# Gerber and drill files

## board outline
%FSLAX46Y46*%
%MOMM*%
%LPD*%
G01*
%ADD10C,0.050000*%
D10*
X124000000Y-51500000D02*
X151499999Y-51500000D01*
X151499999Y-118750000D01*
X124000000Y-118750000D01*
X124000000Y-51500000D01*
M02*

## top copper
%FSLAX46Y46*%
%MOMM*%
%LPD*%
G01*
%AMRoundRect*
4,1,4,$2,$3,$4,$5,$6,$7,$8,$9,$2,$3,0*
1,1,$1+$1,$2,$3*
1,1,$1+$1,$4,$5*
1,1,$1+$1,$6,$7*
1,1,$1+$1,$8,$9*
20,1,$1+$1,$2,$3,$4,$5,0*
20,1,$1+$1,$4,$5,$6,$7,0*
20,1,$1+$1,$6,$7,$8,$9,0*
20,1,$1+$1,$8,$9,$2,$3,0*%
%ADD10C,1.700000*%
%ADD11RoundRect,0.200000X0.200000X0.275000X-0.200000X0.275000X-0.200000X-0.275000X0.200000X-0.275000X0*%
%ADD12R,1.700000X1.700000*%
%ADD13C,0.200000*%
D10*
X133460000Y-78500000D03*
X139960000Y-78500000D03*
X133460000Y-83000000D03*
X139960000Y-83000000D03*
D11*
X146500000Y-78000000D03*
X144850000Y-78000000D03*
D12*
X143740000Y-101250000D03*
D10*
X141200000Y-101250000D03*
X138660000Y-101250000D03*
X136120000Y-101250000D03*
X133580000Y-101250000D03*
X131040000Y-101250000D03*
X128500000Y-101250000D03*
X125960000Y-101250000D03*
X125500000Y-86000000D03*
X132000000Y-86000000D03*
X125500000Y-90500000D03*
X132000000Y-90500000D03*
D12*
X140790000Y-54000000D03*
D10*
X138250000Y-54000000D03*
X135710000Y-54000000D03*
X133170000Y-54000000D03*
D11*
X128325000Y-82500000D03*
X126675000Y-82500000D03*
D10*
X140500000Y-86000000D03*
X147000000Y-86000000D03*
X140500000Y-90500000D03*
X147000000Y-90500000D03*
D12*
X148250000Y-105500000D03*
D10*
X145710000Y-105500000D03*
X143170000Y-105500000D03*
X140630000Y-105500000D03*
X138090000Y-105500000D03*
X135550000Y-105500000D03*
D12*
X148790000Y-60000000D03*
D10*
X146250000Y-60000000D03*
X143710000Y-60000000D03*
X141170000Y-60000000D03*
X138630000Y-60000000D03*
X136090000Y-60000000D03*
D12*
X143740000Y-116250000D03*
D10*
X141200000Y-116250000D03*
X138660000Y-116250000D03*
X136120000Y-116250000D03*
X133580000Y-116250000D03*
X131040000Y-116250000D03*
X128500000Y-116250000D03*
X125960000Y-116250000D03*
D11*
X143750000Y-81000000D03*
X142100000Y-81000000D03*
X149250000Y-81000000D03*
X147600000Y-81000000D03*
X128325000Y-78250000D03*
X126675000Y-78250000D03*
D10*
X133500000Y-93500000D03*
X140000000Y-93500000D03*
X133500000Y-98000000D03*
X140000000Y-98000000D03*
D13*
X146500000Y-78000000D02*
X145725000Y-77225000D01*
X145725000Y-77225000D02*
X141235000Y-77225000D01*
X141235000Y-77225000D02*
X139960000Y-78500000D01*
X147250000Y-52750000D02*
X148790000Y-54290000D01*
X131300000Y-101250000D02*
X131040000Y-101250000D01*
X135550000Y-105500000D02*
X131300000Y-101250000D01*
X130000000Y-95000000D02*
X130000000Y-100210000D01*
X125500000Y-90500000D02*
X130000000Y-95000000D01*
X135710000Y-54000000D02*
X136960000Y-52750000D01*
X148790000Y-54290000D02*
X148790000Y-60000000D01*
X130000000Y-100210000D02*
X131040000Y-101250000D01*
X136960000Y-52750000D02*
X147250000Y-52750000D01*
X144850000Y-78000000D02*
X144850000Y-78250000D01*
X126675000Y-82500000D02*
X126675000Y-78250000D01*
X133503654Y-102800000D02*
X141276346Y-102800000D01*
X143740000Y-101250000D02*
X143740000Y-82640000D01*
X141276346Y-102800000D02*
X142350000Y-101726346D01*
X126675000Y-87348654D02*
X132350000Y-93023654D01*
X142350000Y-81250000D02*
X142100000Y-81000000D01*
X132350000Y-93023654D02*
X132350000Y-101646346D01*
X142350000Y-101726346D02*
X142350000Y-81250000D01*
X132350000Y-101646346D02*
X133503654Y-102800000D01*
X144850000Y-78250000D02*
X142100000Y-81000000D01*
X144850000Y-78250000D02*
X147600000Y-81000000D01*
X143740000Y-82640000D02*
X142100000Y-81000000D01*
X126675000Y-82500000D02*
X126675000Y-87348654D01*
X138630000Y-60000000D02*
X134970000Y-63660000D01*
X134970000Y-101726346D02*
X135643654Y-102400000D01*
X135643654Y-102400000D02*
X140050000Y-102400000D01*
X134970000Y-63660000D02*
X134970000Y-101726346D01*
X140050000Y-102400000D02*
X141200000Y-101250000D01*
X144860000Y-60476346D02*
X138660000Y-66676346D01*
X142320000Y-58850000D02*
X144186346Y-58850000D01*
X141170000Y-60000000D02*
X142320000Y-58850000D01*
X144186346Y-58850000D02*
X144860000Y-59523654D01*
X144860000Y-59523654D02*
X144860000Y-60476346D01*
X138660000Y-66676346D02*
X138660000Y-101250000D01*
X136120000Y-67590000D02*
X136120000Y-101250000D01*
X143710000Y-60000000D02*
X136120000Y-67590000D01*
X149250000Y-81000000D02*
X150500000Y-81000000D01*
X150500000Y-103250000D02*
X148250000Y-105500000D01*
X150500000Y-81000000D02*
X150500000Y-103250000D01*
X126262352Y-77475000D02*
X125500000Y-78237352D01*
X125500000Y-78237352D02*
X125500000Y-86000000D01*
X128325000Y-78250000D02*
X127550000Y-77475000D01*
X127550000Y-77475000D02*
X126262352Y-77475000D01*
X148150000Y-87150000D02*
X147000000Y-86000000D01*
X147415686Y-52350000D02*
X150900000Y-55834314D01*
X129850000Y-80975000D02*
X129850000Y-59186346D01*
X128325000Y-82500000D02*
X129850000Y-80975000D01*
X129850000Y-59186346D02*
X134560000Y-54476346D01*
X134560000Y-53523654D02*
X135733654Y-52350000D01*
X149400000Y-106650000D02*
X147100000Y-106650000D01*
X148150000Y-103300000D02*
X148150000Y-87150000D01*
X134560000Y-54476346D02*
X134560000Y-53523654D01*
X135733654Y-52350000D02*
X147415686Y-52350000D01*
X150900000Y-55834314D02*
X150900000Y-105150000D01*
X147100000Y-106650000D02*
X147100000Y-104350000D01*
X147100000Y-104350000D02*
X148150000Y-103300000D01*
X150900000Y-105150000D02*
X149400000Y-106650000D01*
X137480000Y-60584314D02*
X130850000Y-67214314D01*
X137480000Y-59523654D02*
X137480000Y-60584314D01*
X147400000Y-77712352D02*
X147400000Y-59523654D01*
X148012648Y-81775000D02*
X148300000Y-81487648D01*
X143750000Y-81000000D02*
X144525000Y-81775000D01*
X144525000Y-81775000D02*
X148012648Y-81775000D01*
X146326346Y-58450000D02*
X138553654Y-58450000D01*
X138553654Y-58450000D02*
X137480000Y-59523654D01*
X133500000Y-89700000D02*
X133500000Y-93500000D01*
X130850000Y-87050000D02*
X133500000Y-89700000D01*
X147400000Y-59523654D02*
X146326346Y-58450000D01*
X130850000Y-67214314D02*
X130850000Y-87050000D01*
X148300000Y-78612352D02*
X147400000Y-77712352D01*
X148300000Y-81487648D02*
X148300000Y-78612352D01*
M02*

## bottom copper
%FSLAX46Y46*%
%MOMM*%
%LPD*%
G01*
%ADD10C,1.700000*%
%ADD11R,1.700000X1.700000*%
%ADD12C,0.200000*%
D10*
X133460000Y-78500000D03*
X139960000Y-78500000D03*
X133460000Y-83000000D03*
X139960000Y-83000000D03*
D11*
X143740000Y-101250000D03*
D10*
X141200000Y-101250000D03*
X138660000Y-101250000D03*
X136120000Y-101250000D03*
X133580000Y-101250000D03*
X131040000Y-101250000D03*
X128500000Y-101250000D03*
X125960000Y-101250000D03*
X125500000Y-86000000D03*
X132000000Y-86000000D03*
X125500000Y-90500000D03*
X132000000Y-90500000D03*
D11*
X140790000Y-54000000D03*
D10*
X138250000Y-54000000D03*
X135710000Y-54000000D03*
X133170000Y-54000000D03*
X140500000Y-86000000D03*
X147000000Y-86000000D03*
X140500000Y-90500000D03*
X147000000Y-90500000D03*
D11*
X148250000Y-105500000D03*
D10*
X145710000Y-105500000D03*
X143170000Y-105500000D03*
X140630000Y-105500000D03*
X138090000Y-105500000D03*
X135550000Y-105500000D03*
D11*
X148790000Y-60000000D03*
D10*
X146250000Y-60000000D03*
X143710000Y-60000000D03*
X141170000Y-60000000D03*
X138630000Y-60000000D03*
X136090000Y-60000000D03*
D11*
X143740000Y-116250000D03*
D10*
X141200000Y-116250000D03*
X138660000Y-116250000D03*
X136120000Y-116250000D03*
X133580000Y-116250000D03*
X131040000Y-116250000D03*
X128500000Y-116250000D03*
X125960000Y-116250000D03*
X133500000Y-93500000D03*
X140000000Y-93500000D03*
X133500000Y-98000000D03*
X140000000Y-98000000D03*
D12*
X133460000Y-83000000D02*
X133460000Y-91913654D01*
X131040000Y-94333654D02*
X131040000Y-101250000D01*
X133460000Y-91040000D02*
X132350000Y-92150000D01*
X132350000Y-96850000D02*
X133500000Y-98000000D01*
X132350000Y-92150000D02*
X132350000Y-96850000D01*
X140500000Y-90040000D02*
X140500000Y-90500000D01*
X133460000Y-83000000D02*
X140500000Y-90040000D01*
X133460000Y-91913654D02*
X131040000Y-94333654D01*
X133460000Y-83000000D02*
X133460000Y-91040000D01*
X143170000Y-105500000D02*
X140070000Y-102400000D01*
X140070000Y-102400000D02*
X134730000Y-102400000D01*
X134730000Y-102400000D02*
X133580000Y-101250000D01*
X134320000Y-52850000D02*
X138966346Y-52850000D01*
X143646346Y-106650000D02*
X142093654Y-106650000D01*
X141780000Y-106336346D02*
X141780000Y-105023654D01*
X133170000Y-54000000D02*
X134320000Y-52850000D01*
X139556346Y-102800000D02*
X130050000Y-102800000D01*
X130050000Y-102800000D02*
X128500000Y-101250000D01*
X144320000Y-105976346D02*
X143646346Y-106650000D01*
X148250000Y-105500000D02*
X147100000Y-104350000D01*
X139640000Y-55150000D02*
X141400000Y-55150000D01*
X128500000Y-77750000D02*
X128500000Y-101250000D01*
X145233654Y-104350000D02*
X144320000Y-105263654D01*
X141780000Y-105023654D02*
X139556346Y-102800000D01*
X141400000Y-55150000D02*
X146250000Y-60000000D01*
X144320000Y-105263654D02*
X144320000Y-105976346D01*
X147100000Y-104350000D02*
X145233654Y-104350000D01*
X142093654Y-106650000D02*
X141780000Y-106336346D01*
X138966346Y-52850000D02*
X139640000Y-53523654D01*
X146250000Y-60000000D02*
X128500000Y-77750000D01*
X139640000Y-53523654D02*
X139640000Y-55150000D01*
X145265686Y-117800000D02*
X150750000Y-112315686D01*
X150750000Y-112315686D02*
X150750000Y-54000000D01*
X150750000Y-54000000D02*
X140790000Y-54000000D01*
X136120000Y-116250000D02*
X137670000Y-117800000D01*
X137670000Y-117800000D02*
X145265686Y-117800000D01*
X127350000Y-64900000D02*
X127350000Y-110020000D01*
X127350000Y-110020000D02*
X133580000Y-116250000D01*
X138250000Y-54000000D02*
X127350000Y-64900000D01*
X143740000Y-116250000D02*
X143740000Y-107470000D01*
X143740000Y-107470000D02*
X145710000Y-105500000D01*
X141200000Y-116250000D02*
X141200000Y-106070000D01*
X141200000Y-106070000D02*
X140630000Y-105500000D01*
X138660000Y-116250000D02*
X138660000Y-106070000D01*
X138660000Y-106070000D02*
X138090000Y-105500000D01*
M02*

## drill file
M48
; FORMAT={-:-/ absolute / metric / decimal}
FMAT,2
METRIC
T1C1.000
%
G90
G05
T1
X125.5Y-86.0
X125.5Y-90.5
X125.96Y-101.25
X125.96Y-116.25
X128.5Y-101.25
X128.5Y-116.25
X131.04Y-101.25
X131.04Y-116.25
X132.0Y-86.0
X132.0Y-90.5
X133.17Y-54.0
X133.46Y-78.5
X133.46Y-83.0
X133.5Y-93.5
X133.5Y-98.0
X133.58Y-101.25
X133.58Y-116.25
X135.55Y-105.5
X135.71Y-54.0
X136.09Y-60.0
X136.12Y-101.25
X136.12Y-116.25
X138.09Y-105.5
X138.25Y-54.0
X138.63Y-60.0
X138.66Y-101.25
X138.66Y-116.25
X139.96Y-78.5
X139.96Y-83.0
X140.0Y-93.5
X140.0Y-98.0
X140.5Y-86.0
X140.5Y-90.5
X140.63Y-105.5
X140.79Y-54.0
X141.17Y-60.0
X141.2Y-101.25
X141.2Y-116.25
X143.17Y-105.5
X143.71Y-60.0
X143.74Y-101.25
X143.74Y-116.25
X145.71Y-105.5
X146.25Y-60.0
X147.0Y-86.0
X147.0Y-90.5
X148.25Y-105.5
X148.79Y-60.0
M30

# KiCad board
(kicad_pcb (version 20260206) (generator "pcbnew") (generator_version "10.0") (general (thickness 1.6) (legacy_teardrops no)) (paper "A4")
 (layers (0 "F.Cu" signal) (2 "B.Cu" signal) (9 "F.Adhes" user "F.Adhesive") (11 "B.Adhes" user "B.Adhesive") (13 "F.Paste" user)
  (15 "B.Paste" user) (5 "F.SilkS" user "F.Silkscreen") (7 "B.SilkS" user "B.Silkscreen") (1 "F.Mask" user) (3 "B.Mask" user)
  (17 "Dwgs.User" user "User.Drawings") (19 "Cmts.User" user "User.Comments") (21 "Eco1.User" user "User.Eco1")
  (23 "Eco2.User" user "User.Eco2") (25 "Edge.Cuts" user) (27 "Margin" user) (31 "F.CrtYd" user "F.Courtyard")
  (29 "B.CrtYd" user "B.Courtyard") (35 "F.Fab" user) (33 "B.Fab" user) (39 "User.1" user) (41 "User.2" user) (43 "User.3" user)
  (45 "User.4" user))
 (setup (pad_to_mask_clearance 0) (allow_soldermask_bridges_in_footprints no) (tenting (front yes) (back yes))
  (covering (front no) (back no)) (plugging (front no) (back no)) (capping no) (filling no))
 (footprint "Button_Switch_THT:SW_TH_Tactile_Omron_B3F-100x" (layer "F.Cu") (at 133.46 78.5)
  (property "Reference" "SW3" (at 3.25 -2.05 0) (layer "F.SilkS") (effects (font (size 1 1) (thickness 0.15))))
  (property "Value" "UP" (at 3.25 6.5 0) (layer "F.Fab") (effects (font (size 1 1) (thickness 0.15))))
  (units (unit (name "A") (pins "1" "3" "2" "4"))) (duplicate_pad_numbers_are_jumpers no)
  (pad "1" thru_hole circle (at 0 0) (size 1.7 1.7) (drill 1) (layers "*.Cu" "*.Mask") (remove_unused_layers no) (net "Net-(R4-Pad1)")
   (thermal_bridge_angle 90))
  (pad "1" thru_hole circle (at 6.5 0) (size 1.7 1.7) (drill 1) (layers "*.Cu" "*.Mask") (remove_unused_layers no) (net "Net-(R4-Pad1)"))
  (pad "2" thru_hole circle (at 0 4.5) (size 1.7 1.7) (drill 1) (layers "*.Cu" "*.Mask") (remove_unused_layers no) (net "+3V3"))
  (pad "2" thru_hole circle (at 6.5 4.5) (size 1.7 1.7) (drill 1) (layers "*.Cu" "*.Mask") (remove_unused_layers no)
   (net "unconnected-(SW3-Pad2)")))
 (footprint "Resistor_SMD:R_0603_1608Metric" (layer "F.Cu") (at 145.675 78 180)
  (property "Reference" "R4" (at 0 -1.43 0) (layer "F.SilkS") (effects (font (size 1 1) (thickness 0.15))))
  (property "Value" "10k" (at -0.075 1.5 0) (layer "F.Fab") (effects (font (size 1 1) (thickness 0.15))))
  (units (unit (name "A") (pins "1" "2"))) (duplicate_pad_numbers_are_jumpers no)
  (pad "1" smd roundrect (at -0.825 0 180) (size 0.8 0.95) (layers "F.Cu" "F.Mask" "F.Paste") (roundrect_rratio 0.25) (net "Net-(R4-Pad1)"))
  (pad "2" smd roundrect (at 0.825 0 180) (size 0.8 0.95) (layers "F.Cu" "F.Mask" "F.Paste") (roundrect_rratio 0.25) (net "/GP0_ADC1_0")))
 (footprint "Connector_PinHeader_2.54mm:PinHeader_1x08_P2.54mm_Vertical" (layer "F.Cu") (at 143.74 101.25 -90)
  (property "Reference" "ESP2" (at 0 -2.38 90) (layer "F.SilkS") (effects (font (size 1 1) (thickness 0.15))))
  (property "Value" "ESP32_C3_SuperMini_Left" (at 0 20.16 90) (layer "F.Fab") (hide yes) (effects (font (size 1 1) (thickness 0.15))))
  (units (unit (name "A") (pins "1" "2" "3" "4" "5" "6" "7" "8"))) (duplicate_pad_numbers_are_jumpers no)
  (pad "1" thru_hole rect (at 0 0 270) (size 1.7 1.7) (drill 1) (layers "*.Cu" "*.Mask") (remove_unused_layers no) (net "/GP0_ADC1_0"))
  (pad "2" thru_hole circle (at 0 2.54 270) (size 1.7 1.7) (drill 1) (layers "*.Cu" "*.Mask") (remove_unused_layers no) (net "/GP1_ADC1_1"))
  (pad "3" thru_hole circle (at 0 5.08 270) (size 1.7 1.7) (drill 1) (layers "*.Cu" "*.Mask") (remove_unused_layers no) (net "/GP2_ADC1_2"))
  (pad "4" thru_hole circle (at 0 7.62 270) (size 1.7 1.7) (drill 1) (layers "*.Cu" "*.Mask") (remove_unused_layers no) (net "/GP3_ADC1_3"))
  (pad "5" thru_hole circle (at 0 10.16 270) (size 1.7 1.7) (drill 1) (layers "*.Cu" "*.Mask") (remove_unused_layers no) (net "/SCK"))
  (pad "6" thru_hole circle (at 0 12.7 270) (size 1.7 1.7) (drill 1) (layers "*.Cu" "*.Mask") (remove_unused_layers no) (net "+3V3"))
  (pad "7" thru_hole circle (at 0 15.24 270) (size 1.7 1.7) (drill 1) (layers "*.Cu" "*.Mask") (remove_unused_layers no) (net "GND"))
  (pad "8" thru_hole circle (at 0 17.78 270) (size 1.7 1.7) (drill 1) (layers "*.Cu" "*.Mask") (remove_unused_layers no)
   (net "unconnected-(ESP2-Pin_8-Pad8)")))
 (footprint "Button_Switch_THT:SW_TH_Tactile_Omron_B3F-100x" (layer "F.Cu") (at 125.5 86)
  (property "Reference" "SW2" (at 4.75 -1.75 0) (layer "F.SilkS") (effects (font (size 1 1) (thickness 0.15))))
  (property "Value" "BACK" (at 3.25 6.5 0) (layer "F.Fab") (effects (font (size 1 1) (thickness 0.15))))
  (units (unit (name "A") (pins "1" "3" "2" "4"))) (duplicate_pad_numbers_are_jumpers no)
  (pad "1" thru_hole circle (at 0 0) (size 1.7 1.7) (drill 1) (layers "*.Cu" "*.Mask") (remove_unused_layers no) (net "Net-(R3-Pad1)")
   (thermal_bridge_angle 90))
  (pad "1" thru_hole circle (at 6.5 0) (size 1.7 1.7) (drill 1) (layers "*.Cu" "*.Mask") (remove_unused_layers no) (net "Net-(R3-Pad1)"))
  (pad "2" thru_hole circle (at 0 4.5) (size 1.7 1.7) (drill 1) (layers "*.Cu" "*.Mask") (remove_unused_layers no) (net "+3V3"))
  (pad "2" thru_hole circle (at 6.5 4.5) (size 1.7 1.7) (drill 1) (layers "*.Cu" "*.Mask") (remove_unused_layers no)
   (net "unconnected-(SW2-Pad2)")))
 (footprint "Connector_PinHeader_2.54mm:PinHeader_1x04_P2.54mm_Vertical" (layer "F.Cu") (at 140.79 54 -90)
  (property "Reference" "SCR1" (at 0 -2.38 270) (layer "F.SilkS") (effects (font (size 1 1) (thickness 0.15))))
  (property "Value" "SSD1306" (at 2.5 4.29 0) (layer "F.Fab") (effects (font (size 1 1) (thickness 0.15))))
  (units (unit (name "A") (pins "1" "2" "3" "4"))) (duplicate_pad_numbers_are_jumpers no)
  (pad "1" thru_hole rect (at 0 0 270) (size 1.7 1.7) (drill 1) (layers "*.Cu" "*.Mask") (remove_unused_layers no) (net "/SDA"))
  (pad "2" thru_hole circle (at 0 2.54 270) (size 1.7 1.7) (drill 1) (layers "*.Cu" "*.Mask") (remove_unused_layers no) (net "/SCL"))
  (pad "3" thru_hole circle (at 0 5.08 270) (size 1.7 1.7) (drill 1) (layers "*.Cu" "*.Mask") (remove_unused_layers no) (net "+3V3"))
  (pad "4" thru_hole circle (at 0 7.62 270) (size 1.7 1.7) (drill 1) (layers "*.Cu" "*.Mask") (remove_unused_layers no) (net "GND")))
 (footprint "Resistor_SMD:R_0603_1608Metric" (layer "F.Cu") (at 127.5 82.5 180)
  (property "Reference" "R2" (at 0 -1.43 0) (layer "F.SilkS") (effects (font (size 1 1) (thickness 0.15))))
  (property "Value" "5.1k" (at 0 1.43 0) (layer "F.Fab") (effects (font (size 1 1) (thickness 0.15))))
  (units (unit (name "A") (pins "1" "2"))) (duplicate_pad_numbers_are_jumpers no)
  (pad "1" smd roundrect (at -0.825 0 180) (size 0.8 0.95) (layers "F.Cu" "F.Mask" "F.Paste") (roundrect_rratio 0.25) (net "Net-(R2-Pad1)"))
  (pad "2" smd roundrect (at 0.825 0 180) (size 0.8 0.95) (layers "F.Cu" "F.Mask" "F.Paste") (roundrect_rratio 0.25) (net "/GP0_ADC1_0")))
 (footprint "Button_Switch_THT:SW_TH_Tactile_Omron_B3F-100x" (layer "F.Cu") (at 140.5 86)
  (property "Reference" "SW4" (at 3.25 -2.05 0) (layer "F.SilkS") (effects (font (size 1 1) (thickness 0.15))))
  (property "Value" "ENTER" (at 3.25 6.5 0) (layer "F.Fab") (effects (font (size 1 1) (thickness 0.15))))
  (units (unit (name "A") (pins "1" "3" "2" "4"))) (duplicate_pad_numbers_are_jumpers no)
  (pad "1" thru_hole circle (at 0 0) (size 1.7 1.7) (drill 1) (layers "*.Cu" "*.Mask") (remove_unused_layers no) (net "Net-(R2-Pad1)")
   (thermal_bridge_angle 90))
  (pad "1" thru_hole circle (at 6.5 0) (size 1.7 1.7) (drill 1) (layers "*.Cu" "*.Mask") (remove_unused_layers no) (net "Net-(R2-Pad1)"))
  (pad "2" thru_hole circle (at 0 4.5) (size 1.7 1.7) (drill 1) (layers "*.Cu" "*.Mask") (remove_unused_layers no) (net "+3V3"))
  (pad "2" thru_hole circle (at 6.5 4.5) (size 1.7 1.7) (drill 1) (layers "*.Cu" "*.Mask") (remove_unused_layers no)
   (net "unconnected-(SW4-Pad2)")))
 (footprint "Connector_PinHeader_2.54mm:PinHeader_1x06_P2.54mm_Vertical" (layer "F.Cu") (at 148.25 105.5 -90)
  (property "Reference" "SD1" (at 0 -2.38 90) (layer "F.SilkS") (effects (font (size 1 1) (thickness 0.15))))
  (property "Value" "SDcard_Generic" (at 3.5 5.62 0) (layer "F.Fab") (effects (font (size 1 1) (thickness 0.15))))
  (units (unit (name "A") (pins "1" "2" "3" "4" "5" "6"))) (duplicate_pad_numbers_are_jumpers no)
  (pad "1" thru_hole rect (at 0 0 270) (size 1.7 1.7) (drill 1) (layers "*.Cu" "*.Mask") (remove_unused_layers no) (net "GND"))
  (pad "2" thru_hole circle (at 0 2.54 270) (size 1.7 1.7) (drill 1) (layers "*.Cu" "*.Mask") (remove_unused_layers no) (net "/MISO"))
  (pad "3" thru_hole circle (at 0 5.08 270) (size 1.7 1.7) (drill 1) (layers "*.Cu" "*.Mask") (remove_unused_layers no) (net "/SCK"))
  (pad "4" thru_hole circle (at 0 7.62 270) (size 1.7 1.7) (drill 1) (layers "*.Cu" "*.Mask") (remove_unused_layers no) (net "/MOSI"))
  (pad "5" thru_hole circle (at 0 10.16 270) (size 1.7 1.7) (drill 1) (layers "*.Cu" "*.Mask") (remove_unused_layers no) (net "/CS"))
  (pad "6" thru_hole circle (at 0 12.7 270) (size 1.7 1.7) (drill 1) (layers "*.Cu" "*.Mask") (remove_unused_layers no) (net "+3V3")))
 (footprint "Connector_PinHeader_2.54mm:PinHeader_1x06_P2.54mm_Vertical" (layer "F.Cu") (at 148.79 60 -90)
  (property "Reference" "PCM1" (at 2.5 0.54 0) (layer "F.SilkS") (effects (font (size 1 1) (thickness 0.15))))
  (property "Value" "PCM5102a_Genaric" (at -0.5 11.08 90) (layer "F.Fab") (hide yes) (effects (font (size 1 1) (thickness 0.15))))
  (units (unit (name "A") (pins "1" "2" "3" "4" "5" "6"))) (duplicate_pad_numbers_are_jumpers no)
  (pad "1" thru_hole rect (at 0 0 270) (size 1.7 1.7) (drill 1) (layers "*.Cu" "*.Mask") (remove_unused_layers no) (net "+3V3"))
  (pad "2" thru_hole circle (at 0 2.54 270) (size 1.7 1.7) (drill 1) (layers "*.Cu" "*.Mask") (remove_unused_layers no) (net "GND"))
  (pad "3" thru_hole circle (at 0 5.08 270) (size 1.7 1.7) (drill 1) (layers "*.Cu" "*.Mask") (remove_unused_layers no) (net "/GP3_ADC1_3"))
  (pad "4" thru_hole circle (at 0 7.62 270) (size 1.7 1.7) (drill 1) (layers "*.Cu" "*.Mask") (remove_unused_layers no) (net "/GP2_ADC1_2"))
  (pad "5" thru_hole circle (at 0 10.16 270) (size 1.7 1.7) (drill 1) (layers "*.Cu" "*.Mask") (remove_unused_layers no) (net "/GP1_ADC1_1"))
  (pad "6" thru_hole circle (at 0 12.7 270) (size 1.7 1.7) (drill 1) (layers "*.Cu" "*.Mask") (remove_unused_layers no)
   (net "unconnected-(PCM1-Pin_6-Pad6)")))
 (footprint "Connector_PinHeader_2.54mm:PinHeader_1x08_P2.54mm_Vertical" (layer "F.Cu") (at 143.74 116.25 -90)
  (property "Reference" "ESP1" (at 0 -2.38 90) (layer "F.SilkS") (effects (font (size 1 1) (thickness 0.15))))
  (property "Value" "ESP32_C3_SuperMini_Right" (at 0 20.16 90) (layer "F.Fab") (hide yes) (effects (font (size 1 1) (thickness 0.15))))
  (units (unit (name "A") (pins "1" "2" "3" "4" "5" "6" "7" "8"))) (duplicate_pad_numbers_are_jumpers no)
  (pad "1" thru_hole rect (at 0 0 270) (size 1.7 1.7) (drill 1) (layers "*.Cu" "*.Mask") (remove_unused_layers no) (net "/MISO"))
  (pad "2" thru_hole circle (at 0 2.54 270) (size 1.7 1.7) (drill 1) (layers "*.Cu" "*.Mask") (remove_unused_layers no) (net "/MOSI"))
  (pad "3" thru_hole circle (at 0 5.08 270) (size 1.7 1.7) (drill 1) (layers "*.Cu" "*.Mask") (remove_unused_layers no) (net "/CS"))
  (pad "4" thru_hole circle (at 0 7.62 270) (size 1.7 1.7) (drill 1) (layers "*.Cu" "*.Mask") (remove_unused_layers no) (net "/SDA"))
  (pad "5" thru_hole circle (at 0 10.16 270) (size 1.7 1.7) (drill 1) (layers "*.Cu" "*.Mask") (remove_unused_layers no) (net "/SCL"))
  (pad "6" thru_hole circle (at 0 12.7 270) (size 1.7 1.7) (drill 1) (layers "*.Cu" "*.Mask") (remove_unused_layers no)
   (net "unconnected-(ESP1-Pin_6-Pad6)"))
  (pad "7" thru_hole circle (at 0 15.24 270) (size 1.7 1.7) (drill 1) (layers "*.Cu" "*.Mask") (remove_unused_layers no)
   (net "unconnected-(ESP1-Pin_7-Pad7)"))
  (pad "8" thru_hole circle (at 0 17.78 270) (size 1.7 1.7) (drill 1) (layers "*.Cu" "*.Mask") (remove_unused_layers no)
   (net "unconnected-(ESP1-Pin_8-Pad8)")))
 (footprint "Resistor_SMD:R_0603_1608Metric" (layer "F.Cu") (at 142.925 81 180)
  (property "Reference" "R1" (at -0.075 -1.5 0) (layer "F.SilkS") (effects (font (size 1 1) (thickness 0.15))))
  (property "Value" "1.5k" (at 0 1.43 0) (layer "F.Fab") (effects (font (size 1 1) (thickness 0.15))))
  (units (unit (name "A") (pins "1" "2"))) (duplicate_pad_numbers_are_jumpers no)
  (pad "1" smd roundrect (at -0.825 0 180) (size 0.8 0.95) (layers "F.Cu" "F.Mask" "F.Paste") (roundrect_rratio 0.25) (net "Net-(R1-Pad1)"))
  (pad "2" smd roundrect (at 0.825 0 180) (size 0.8 0.95) (layers "F.Cu" "F.Mask" "F.Paste") (roundrect_rratio 0.25) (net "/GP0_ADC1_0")))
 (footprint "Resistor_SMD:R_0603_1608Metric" (layer "F.Cu") (at 148.425 81 180)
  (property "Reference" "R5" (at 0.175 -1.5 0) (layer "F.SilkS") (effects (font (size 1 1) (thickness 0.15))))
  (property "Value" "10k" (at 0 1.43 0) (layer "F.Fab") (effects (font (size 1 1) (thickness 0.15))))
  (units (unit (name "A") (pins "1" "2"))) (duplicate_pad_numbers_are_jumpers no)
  (pad "1" smd roundrect (at -0.825 0 180) (size 0.8 0.95) (layers "F.Cu" "F.Mask" "F.Paste") (roundrect_rratio 0.25) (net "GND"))
  (pad "2" smd roundrect (at 0.825 0 180) (size 0.8 0.95) (layers "F.Cu" "F.Mask" "F.Paste") (roundrect_rratio 0.25) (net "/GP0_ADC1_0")))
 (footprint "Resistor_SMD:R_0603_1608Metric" (layer "F.Cu") (at 127.5 78.25 180)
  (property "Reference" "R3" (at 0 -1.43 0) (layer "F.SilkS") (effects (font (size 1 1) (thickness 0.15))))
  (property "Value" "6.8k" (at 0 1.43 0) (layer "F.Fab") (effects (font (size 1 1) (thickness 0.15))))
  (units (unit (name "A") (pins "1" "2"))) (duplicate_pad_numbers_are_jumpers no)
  (pad "1" smd roundrect (at -0.825 0 180) (size 0.8 0.95) (layers "F.Cu" "F.Mask" "F.Paste") (roundrect_rratio 0.25) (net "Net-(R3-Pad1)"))
  (pad "2" smd roundrect (at 0.825 0 180) (size 0.8 0.95) (layers "F.Cu" "F.Mask" "F.Paste") (roundrect_rratio 0.25) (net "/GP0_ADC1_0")))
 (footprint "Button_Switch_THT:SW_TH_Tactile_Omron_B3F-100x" (layer "F.Cu") (at 133.5 93.5)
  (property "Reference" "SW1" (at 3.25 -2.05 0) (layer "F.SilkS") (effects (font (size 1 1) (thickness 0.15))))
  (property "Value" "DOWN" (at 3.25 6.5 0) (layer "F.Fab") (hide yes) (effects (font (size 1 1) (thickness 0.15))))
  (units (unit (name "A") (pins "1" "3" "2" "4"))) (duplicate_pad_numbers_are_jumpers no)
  (pad "1" thru_hole circle (at 0 0) (size 1.7 1.7) (drill 1) (layers "*.Cu" "*.Mask") (remove_unused_layers no) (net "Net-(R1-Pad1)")
   (thermal_bridge_angle 90))
  (pad "1" thru_hole circle (at 6.5 0) (size 1.7 1.7) (drill 1) (layers "*.Cu" "*.Mask") (remove_unused_layers no) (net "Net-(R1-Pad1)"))
  (pad "2" thru_hole circle (at 0 4.5) (size 1.7 1.7) (drill 1) (layers "*.Cu" "*.Mask") (remove_unused_layers no) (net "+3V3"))
  (pad "2" thru_hole circle (at 6.5 4.5) (size 1.7 1.7) (drill 1) (layers "*.Cu" "*.Mask") (remove_unused_layers no)
   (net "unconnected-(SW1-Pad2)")))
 (gr_rect (start 124 51.5) (end 151.499999 118.75) (stroke (width 0.05) (type default)) (fill no) (layer "Edge.Cuts"))
 (segment (start 146.5 78) (end 145.725 77.225) (width 0.2) (layer "F.Cu") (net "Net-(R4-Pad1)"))
 (segment (start 145.725 77.225) (end 141.235 77.225) (width 0.2) (layer "F.Cu") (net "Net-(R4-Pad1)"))
 (segment (start 141.235 77.225) (end 139.96 78.5) (width 0.2) (layer "F.Cu") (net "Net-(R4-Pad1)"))
 (segment (start 147.25 52.75) (end 148.79 54.29) (width 0.2) (layer "F.Cu") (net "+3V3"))
 (segment (start 131.3 101.25) (end 131.04 101.25) (width 0.2) (layer "F.Cu") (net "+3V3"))
 (segment (start 135.55 105.5) (end 131.3 101.25) (width 0.2) (layer "F.Cu") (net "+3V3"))
 (segment (start 130 95) (end 130 100.21) (width 0.2) (layer "F.Cu") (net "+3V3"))
 (segment (start 125.5 90.5) (end 130 95) (width 0.2) (layer "F.Cu") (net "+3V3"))
 (segment (start 135.71 54) (end 136.96 52.75) (width 0.2) (layer "F.Cu") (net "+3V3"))
 (segment (start 148.79 54.29) (end 148.79 60) (width 0.2) (layer "F.Cu") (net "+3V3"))
 (segment (start 130 100.21) (end 131.04 101.25) (width 0.2) (layer "F.Cu") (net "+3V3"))
 (segment (start 136.96 52.75) (end 147.25 52.75) (width 0.2) (layer "F.Cu") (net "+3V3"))
 (segment (start 133.46 83) (end 133.46 91.913654) (width 0.2) (layer "B.Cu") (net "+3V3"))
 (segment (start 131.04 94.333654) (end 131.04 101.25) (width 0.2) (layer "B.Cu") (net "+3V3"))
 (segment (start 133.46 91.04) (end 132.35 92.15) (width 0.2) (layer "B.Cu") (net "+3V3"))
 (segment (start 132.35 96.85) (end 133.5 98) (width 0.2) (layer "B.Cu") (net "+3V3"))
 (segment (start 132.35 92.15) (end 132.35 96.85) (width 0.2) (layer "B.Cu") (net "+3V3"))
 (segment (start 140.5 90.04) (end 140.5 90.5) (width 0.2) (layer "B.Cu") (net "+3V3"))
 (segment (start 133.46 83) (end 140.5 90.04) (width 0.2) (layer "B.Cu") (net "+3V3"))
 (segment (start 133.46 91.913654) (end 131.04 94.333654) (width 0.2) (layer "B.Cu") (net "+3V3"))
 (segment (start 133.46 83) (end 133.46 91.04) (width 0.2) (layer "B.Cu") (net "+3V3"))
 (segment (start 144.85 78) (end 144.85 78.25) (width 0.2) (layer "F.Cu") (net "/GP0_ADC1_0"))
 (segment (start 126.675 82.5) (end 126.675 78.25) (width 0.2) (layer "F.Cu") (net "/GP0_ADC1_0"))
 (segment (start 133.503654 102.8) (end 141.276346 102.8) (width 0.2) (layer "F.Cu") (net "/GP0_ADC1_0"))
 (segment (start 143.74 101.25) (end 143.74 82.64) (width 0.2) (layer "F.Cu") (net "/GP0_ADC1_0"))
 (segment (start 141.276346 102.8) (end 142.35 101.726346) (width 0.2) (layer "F.Cu") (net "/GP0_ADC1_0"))
 (segment (start 126.675 87.348654) (end 132.35 93.023654) (width 0.2) (layer "F.Cu") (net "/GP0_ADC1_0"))
 (segment (start 142.35 81.25) (end 142.1 81) (width 0.2) (layer "F.Cu") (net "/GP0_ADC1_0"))
 (segment (start 132.35 93.023654) (end 132.35 101.646346) (width 0.2) (layer "F.Cu") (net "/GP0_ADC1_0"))
 (segment (start 142.35 101.726346) (end 142.35 81.25) (width 0.2) (layer "F.Cu") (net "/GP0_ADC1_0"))
 (segment (start 132.35 101.646346) (end 133.503654 102.8) (width 0.2) (layer "F.Cu") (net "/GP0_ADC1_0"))
 (segment (start 144.85 78.25) (end 142.1 81) (width 0.2) (layer "F.Cu") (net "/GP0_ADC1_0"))
 (segment (start 144.85 78.25) (end 147.6 81) (width 0.2) (layer "F.Cu") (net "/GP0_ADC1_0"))
 (segment (start 143.74 82.64) (end 142.1 81) (width 0.2) (layer "F.Cu") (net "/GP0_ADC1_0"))
 (segment (start 126.675 82.5) (end 126.675 87.348654) (width 0.2) (layer "F.Cu") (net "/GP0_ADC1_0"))
 (segment (start 138.63 60) (end 134.97 63.66) (width 0.2) (layer "F.Cu") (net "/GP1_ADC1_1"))
 (segment (start 134.97 101.726346) (end 135.643654 102.4) (width 0.2) (layer "F.Cu") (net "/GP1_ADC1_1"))
 (segment (start 135.643654 102.4) (end 140.05 102.4) (width 0.2) (layer "F.Cu") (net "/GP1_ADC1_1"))
 (segment (start 134.97 63.66) (end 134.97 101.726346) (width 0.2) (layer "F.Cu") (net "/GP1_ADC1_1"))
 (segment (start 140.05 102.4) (end 141.2 101.25) (width 0.2) (layer "F.Cu") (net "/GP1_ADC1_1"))
 (segment (start 144.86 60.476346) (end 138.66 66.676346) (width 0.2) (layer "F.Cu") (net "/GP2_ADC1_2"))
 (segment (start 142.32 58.85) (end 144.186346 58.85) (width 0.2) (layer "F.Cu") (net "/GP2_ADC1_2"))
 (segment (start 141.17 60) (end 142.32 58.85) (width 0.2) (layer "F.Cu") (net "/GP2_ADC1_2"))
 (segment (start 144.186346 58.85) (end 144.86 59.523654) (width 0.2) (layer "F.Cu") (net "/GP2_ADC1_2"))
 (segment (start 144.86 59.523654) (end 144.86 60.476346) (width 0.2) (layer "F.Cu") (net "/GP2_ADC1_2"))
 (segment (start 138.66 66.676346) (end 138.66 101.25) (width 0.2) (layer "F.Cu") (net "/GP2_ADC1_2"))
 (segment (start 136.12 67.59) (end 136.12 101.25) (width 0.2) (layer "F.Cu") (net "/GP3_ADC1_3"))
 (segment (start 143.71 60) (end 136.12 67.59) (width 0.2) (layer "F.Cu") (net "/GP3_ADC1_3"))
 (segment (start 143.17 105.5) (end 140.07 102.4) (width 0.2) (layer "B.Cu") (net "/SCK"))
 (segment (start 140.07 102.4) (end 134.73 102.4) (width 0.2) (layer "B.Cu") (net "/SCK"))
 (segment (start 134.73 102.4) (end 133.58 101.25) (width 0.2) (layer "B.Cu") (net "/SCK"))
 (segment (start 149.25 81) (end 150.5 81) (width 0.2) (layer "F.Cu") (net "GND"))
 (segment (start 150.5 103.25) (end 148.25 105.5) (width 0.2) (layer "F.Cu") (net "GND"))
 (segment (start 150.5 81) (end 150.5 103.25) (width 0.2) (layer "F.Cu") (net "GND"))
 (segment (start 134.32 52.85) (end 138.966346 52.85) (width 0.2) (layer "B.Cu") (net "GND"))
 (segment (start 143.646346 106.65) (end 142.093654 106.65) (width 0.2) (layer "B.Cu") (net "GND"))
 (segment (start 141.78 106.336346) (end 141.78 105.023654) (width 0.2) (layer "B.Cu") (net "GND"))
 (segment (start 133.17 54) (end 134.32 52.85) (width 0.2) (layer "B.Cu") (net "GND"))
 (segment (start 139.556346 102.8) (end 130.05 102.8) (width 0.2) (layer "B.Cu") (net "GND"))
 (segment (start 130.05 102.8) (end 128.5 101.25) (width 0.2) (layer "B.Cu") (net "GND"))
 (segment (start 144.32 105.976346) (end 143.646346 106.65) (width 0.2) (layer "B.Cu") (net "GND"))
 (segment (start 148.25 105.5) (end 147.1 104.35) (width 0.2) (layer "B.Cu") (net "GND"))
 (segment (start 139.64 55.15) (end 141.4 55.15) (width 0.2) (layer "B.Cu") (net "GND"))
 (segment (start 128.5 77.75) (end 128.5 101.25) (width 0.2) (layer "B.Cu") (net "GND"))
 (segment (start 145.233654 104.35) (end 144.32 105.263654) (width 0.2) (layer "B.Cu") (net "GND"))
 (segment (start 141.78 105.023654) (end 139.556346 102.8) (width 0.2) (layer "B.Cu") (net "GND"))
 (segment (start 141.4 55.15) (end 146.25 60) (width 0.2) (layer "B.Cu") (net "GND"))
 (segment (start 144.32 105.263654) (end 144.32 105.976346) (width 0.2) (layer "B.Cu") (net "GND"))
 (segment (start 147.1 104.35) (end 145.233654 104.35) (width 0.2) (layer "B.Cu") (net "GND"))
 (segment (start 142.093654 106.65) (end 141.78 106.336346) (width 0.2) (layer "B.Cu") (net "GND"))
 (segment (start 138.966346 52.85) (end 139.64 53.523654) (width 0.2) (layer "B.Cu") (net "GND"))
 (segment (start 146.25 60) (end 128.5 77.75) (width 0.2) (layer "B.Cu") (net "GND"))
 (segment (start 139.64 53.523654) (end 139.64 55.15) (width 0.2) (layer "B.Cu") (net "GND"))
 (segment (start 126.262352 77.475) (end 125.5 78.237352) (width 0.2) (layer "F.Cu") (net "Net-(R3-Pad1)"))
 (segment (start 125.5 78.237352) (end 125.5 86) (width 0.2) (layer "F.Cu") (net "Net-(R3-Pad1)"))
 (segment (start 128.325 78.25) (end 127.55 77.475) (width 0.2) (layer "F.Cu") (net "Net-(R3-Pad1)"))
 (segment (start 127.55 77.475) (end 126.262352 77.475) (width 0.2) (layer "F.Cu") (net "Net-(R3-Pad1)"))
 (segment (start 145.265686 117.8) (end 150.75 112.315686) (width 0.2) (layer "B.Cu") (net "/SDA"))
 (segment (start 150.75 112.315686) (end 150.75 54) (width 0.2) (layer "B.Cu") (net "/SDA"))
 (segment (start 150.75 54) (end 140.79 54) (width 0.2) (layer "B.Cu") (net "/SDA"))
 (segment (start 136.12 116.25) (end 137.67 117.8) (width 0.2) (layer "B.Cu") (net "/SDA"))
 (segment (start 137.67 117.8) (end 145.265686 117.8) (width 0.2) (layer "B.Cu") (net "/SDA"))
 (segment (start 127.35 64.9) (end 127.35 110.02) (width 0.2) (layer "B.Cu") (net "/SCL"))
 (segment (start 127.35 110.02) (end 133.58 116.25) (width 0.2) (layer "B.Cu") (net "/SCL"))
 (segment (start 138.25 54) (end 127.35 64.9) (width 0.2) (layer "B.Cu") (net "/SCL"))
 (segment (start 148.15 87.15) (end 147 86) (width 0.2) (layer "F.Cu") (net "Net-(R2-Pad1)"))
 (segment (start 147.415686 52.35) (end 150.9 55.834314) (width 0.2) (layer "F.Cu") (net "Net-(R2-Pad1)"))
 (segment (start 129.85 80.975) (end 129.85 59.186346) (width 0.2) (layer "F.Cu") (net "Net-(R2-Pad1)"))
 (segment (start 128.325 82.5) (end 129.85 80.975) (width 0.2) (layer "F.Cu") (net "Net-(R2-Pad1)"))
 (segment (start 129.85 59.186346) (end 134.56 54.476346) (width 0.2) (layer "F.Cu") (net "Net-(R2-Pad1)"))
 (segment (start 134.56 53.523654) (end 135.733654 52.35) (width 0.2) (layer "F.Cu") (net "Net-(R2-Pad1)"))
 (segment (start 149.4 106.65) (end 147.1 106.65) (width 0.2) (layer "F.Cu") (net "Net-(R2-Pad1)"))
 (segment (start 148.15 103.3) (end 148.15 87.15) (width 0.2) (layer "F.Cu") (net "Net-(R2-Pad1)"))
 (segment (start 134.56 54.476346) (end 134.56 53.523654) (width 0.2) (layer "F.Cu") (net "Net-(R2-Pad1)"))
 (segment (start 135.733654 52.35) (end 147.415686 52.35) (width 0.2) (layer "F.Cu") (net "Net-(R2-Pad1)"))
 (segment (start 150.9 55.834314) (end 150.9 105.15) (width 0.2) (layer "F.Cu") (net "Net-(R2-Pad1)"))
 (segment (start 147.1 106.65) (end 147.1 104.35) (width 0.2) (layer "F.Cu") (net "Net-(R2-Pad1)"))
 (segment (start 147.1 104.35) (end 148.15 103.3) (width 0.2) (layer "F.Cu") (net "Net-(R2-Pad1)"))
 (segment (start 150.9 105.15) (end 149.4 106.65) (width 0.2) (layer "F.Cu") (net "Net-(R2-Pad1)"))
 (segment (start 143.74 116.25) (end 143.74 107.47) (width 0.2) (layer "B.Cu") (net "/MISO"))
 (segment (start 143.74 107.47) (end 145.71 105.5) (width 0.2) (layer "B.Cu") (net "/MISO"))
 (segment (start 141.2 116.25) (end 141.2 106.07) (width 0.2) (layer "B.Cu") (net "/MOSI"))
 (segment (start 141.2 106.07) (end 140.63 105.5) (width 0.2) (layer "B.Cu") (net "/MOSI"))
 (segment (start 138.66 116.25) (end 138.66 106.07) (width 0.2) (layer "B.Cu") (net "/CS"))
 (segment (start 138.66 106.07) (end 138.09 105.5) (width 0.2) (layer "B.Cu") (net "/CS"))
 (segment (start 137.48 60.584314) (end 130.85 67.214314) (width 0.2) (layer "F.Cu") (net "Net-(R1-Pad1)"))
 (segment (start 137.48 59.523654) (end 137.48 60.584314) (width 0.2) (layer "F.Cu") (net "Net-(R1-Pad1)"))
 (segment (start 147.4 77.712352) (end 147.4 59.523654) (width 0.2) (layer "F.Cu") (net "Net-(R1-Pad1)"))
 (segment (start 148.012648 81.775) (end 148.3 81.487648) (width 0.2) (layer "F.Cu") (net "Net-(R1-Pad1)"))
 (segment (start 143.75 81) (end 144.525 81.775) (width 0.2) (layer "F.Cu") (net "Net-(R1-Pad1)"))
 (segment (start 144.525 81.775) (end 148.012648 81.775) (width 0.2) (layer "F.Cu") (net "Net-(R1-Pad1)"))
 (segment (start 146.326346 58.45) (end 138.553654 58.45) (width 0.2) (layer "F.Cu") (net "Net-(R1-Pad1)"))
 (segment (start 138.553654 58.45) (end 137.48 59.523654) (width 0.2) (layer "F.Cu") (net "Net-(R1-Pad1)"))
 (segment (start 133.5 89.7) (end 133.5 93.5) (width 0.2) (layer "F.Cu") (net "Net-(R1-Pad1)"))
 (segment (start 130.85 87.05) (end 133.5 89.7) (width 0.2) (layer "F.Cu") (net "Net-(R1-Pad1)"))
 (segment (start 147.4 59.523654) (end 146.326346 58.45) (width 0.2) (layer "F.Cu") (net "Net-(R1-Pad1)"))
 (segment (start 130.85 67.214314) (end 130.85 87.05) (width 0.2) (layer "F.Cu") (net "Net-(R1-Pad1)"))
 (segment (start 148.3 78.612352) (end 147.4 77.712352) (width 0.2) (layer "F.Cu") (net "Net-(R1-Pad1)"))
 (segment (start 148.3 81.487648) (end 148.3 78.612352) (width 0.2) (layer "F.Cu") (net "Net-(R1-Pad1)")))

